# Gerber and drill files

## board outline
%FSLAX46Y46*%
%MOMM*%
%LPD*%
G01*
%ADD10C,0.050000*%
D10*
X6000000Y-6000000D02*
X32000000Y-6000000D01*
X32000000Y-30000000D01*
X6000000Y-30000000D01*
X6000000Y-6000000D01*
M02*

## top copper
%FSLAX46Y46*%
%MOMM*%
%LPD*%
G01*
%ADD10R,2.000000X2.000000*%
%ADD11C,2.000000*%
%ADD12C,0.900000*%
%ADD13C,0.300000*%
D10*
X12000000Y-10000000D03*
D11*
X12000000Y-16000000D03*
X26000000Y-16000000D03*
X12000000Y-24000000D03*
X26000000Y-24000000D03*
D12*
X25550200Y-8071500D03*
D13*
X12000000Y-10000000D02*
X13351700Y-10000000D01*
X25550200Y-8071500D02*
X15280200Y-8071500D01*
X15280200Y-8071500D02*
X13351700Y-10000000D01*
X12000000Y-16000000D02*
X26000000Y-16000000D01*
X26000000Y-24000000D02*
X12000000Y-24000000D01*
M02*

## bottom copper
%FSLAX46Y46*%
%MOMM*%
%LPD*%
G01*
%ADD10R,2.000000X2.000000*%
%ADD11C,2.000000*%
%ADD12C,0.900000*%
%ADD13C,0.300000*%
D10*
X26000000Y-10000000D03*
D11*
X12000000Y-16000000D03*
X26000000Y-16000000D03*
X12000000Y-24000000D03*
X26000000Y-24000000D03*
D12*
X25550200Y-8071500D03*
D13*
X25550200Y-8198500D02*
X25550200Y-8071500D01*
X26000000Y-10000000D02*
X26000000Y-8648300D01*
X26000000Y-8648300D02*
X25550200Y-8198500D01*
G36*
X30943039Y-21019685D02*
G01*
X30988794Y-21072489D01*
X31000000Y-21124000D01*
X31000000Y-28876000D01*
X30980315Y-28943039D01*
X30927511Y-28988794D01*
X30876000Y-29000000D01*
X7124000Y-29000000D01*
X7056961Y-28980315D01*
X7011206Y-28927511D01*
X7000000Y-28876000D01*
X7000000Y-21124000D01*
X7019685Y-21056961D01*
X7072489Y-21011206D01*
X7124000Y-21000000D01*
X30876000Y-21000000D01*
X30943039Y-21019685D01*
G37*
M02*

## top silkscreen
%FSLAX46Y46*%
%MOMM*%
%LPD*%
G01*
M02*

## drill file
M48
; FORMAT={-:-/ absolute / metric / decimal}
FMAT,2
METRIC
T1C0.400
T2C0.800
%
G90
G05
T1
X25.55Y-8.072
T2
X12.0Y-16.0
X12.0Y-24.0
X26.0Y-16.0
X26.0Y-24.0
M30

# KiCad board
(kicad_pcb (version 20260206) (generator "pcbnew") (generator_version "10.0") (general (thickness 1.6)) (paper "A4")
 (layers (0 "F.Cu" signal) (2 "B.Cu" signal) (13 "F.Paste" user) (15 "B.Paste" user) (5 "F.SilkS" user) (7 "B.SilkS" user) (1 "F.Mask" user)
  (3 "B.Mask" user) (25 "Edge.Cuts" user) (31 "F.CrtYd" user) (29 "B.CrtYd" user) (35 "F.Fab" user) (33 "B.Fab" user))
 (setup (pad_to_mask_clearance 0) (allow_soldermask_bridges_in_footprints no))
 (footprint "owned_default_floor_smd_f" (layer "F.Cu") (at 12 10)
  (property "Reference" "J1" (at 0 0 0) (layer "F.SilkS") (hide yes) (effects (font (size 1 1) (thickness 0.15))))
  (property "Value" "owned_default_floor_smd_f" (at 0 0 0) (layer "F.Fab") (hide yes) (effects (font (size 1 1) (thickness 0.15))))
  (pad "1" smd rect (at 0 0) (size 2 2) (layers "F.Cu" "F.Paste" "F.Mask") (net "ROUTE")))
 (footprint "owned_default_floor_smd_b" (layer "B.Cu") (at 26 10)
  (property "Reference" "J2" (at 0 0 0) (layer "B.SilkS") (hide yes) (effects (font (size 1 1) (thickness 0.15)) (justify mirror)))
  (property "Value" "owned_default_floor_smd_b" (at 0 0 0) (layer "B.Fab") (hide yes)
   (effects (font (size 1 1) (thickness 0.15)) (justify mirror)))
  (pad "1" smd rect (at 0 0) (size 2 2) (layers "B.Cu" "B.Paste" "B.Mask") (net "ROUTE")))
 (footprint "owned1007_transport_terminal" (layer "F.Cu") (at 12 16)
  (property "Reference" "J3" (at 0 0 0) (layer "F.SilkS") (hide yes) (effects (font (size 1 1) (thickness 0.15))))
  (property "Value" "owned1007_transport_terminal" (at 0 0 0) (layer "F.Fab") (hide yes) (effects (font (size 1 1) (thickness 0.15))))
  (pad "1" thru_hole circle (at 0 0) (size 2 2) (drill 0.8) (layers "*.Cu" "*.Mask") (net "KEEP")))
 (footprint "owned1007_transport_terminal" (layer "F.Cu") (at 26 16)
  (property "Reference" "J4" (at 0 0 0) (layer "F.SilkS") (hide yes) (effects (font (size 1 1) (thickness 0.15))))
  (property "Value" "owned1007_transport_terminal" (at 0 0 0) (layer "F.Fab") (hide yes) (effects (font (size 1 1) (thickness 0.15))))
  (pad "1" thru_hole circle (at 0 0) (size 2 2) (drill 0.8) (layers "*.Cu" "*.Mask") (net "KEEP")))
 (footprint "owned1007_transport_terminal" (layer "F.Cu") (at 12 24)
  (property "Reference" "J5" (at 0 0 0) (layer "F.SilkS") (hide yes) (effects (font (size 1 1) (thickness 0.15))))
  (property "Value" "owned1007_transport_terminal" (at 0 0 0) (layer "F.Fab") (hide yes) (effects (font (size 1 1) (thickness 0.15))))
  (pad "1" thru_hole circle (at 0 0) (size 2 2) (drill 0.8) (layers "*.Cu" "*.Mask") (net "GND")))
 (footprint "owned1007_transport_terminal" (layer "F.Cu") (at 26 24)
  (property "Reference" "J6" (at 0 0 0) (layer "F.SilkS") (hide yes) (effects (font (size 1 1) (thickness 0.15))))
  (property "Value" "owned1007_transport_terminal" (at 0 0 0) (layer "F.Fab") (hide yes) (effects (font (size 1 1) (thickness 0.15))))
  (pad "1" thru_hole circle (at 0 0) (size 2 2) (drill 0.8) (layers "*.Cu" "*.Mask") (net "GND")))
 (gr_rect (start 6 6) (end 32 30) (stroke (width 0.05) (type default)) (fill none) (layer "Edge.Cuts"))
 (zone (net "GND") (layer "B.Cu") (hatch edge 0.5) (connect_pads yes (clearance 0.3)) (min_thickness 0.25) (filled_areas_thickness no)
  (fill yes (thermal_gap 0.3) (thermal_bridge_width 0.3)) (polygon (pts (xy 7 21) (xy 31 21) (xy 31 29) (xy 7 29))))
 (segment (start 12 10) (end 13.3517 10) (width 0.3) (layer "F.Cu") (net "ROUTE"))
 (segment (start 25.5502 8.0715) (end 15.2802 8.0715) (width 0.3) (layer "F.Cu") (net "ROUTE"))
 (segment (start 15.2802 8.0715) (end 13.3517 10) (width 0.3) (layer "F.Cu") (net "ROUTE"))
 (via (at 25.5502 8.0715) (size 0.9) (drill 0.4) (layers "F.Cu" "B.Cu") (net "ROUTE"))
 (segment (start 25.5502 8.1985) (end 25.5502 8.0715) (width 0.3) (layer "B.Cu") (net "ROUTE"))
 (segment (start 26 10) (end 26 8.6483) (width 0.3) (layer "B.Cu") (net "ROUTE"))
 (segment (start 26 8.6483) (end 25.5502 8.1985) (width 0.3) (layer "B.Cu") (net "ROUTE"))
 (segment (start 12 16) (end 26 16) (width 0.3) (layer "F.Cu") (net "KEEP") (locked yes))
 (segment (start 26 24) (end 12 24) (width 0.3) (layer "F.Cu") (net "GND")))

